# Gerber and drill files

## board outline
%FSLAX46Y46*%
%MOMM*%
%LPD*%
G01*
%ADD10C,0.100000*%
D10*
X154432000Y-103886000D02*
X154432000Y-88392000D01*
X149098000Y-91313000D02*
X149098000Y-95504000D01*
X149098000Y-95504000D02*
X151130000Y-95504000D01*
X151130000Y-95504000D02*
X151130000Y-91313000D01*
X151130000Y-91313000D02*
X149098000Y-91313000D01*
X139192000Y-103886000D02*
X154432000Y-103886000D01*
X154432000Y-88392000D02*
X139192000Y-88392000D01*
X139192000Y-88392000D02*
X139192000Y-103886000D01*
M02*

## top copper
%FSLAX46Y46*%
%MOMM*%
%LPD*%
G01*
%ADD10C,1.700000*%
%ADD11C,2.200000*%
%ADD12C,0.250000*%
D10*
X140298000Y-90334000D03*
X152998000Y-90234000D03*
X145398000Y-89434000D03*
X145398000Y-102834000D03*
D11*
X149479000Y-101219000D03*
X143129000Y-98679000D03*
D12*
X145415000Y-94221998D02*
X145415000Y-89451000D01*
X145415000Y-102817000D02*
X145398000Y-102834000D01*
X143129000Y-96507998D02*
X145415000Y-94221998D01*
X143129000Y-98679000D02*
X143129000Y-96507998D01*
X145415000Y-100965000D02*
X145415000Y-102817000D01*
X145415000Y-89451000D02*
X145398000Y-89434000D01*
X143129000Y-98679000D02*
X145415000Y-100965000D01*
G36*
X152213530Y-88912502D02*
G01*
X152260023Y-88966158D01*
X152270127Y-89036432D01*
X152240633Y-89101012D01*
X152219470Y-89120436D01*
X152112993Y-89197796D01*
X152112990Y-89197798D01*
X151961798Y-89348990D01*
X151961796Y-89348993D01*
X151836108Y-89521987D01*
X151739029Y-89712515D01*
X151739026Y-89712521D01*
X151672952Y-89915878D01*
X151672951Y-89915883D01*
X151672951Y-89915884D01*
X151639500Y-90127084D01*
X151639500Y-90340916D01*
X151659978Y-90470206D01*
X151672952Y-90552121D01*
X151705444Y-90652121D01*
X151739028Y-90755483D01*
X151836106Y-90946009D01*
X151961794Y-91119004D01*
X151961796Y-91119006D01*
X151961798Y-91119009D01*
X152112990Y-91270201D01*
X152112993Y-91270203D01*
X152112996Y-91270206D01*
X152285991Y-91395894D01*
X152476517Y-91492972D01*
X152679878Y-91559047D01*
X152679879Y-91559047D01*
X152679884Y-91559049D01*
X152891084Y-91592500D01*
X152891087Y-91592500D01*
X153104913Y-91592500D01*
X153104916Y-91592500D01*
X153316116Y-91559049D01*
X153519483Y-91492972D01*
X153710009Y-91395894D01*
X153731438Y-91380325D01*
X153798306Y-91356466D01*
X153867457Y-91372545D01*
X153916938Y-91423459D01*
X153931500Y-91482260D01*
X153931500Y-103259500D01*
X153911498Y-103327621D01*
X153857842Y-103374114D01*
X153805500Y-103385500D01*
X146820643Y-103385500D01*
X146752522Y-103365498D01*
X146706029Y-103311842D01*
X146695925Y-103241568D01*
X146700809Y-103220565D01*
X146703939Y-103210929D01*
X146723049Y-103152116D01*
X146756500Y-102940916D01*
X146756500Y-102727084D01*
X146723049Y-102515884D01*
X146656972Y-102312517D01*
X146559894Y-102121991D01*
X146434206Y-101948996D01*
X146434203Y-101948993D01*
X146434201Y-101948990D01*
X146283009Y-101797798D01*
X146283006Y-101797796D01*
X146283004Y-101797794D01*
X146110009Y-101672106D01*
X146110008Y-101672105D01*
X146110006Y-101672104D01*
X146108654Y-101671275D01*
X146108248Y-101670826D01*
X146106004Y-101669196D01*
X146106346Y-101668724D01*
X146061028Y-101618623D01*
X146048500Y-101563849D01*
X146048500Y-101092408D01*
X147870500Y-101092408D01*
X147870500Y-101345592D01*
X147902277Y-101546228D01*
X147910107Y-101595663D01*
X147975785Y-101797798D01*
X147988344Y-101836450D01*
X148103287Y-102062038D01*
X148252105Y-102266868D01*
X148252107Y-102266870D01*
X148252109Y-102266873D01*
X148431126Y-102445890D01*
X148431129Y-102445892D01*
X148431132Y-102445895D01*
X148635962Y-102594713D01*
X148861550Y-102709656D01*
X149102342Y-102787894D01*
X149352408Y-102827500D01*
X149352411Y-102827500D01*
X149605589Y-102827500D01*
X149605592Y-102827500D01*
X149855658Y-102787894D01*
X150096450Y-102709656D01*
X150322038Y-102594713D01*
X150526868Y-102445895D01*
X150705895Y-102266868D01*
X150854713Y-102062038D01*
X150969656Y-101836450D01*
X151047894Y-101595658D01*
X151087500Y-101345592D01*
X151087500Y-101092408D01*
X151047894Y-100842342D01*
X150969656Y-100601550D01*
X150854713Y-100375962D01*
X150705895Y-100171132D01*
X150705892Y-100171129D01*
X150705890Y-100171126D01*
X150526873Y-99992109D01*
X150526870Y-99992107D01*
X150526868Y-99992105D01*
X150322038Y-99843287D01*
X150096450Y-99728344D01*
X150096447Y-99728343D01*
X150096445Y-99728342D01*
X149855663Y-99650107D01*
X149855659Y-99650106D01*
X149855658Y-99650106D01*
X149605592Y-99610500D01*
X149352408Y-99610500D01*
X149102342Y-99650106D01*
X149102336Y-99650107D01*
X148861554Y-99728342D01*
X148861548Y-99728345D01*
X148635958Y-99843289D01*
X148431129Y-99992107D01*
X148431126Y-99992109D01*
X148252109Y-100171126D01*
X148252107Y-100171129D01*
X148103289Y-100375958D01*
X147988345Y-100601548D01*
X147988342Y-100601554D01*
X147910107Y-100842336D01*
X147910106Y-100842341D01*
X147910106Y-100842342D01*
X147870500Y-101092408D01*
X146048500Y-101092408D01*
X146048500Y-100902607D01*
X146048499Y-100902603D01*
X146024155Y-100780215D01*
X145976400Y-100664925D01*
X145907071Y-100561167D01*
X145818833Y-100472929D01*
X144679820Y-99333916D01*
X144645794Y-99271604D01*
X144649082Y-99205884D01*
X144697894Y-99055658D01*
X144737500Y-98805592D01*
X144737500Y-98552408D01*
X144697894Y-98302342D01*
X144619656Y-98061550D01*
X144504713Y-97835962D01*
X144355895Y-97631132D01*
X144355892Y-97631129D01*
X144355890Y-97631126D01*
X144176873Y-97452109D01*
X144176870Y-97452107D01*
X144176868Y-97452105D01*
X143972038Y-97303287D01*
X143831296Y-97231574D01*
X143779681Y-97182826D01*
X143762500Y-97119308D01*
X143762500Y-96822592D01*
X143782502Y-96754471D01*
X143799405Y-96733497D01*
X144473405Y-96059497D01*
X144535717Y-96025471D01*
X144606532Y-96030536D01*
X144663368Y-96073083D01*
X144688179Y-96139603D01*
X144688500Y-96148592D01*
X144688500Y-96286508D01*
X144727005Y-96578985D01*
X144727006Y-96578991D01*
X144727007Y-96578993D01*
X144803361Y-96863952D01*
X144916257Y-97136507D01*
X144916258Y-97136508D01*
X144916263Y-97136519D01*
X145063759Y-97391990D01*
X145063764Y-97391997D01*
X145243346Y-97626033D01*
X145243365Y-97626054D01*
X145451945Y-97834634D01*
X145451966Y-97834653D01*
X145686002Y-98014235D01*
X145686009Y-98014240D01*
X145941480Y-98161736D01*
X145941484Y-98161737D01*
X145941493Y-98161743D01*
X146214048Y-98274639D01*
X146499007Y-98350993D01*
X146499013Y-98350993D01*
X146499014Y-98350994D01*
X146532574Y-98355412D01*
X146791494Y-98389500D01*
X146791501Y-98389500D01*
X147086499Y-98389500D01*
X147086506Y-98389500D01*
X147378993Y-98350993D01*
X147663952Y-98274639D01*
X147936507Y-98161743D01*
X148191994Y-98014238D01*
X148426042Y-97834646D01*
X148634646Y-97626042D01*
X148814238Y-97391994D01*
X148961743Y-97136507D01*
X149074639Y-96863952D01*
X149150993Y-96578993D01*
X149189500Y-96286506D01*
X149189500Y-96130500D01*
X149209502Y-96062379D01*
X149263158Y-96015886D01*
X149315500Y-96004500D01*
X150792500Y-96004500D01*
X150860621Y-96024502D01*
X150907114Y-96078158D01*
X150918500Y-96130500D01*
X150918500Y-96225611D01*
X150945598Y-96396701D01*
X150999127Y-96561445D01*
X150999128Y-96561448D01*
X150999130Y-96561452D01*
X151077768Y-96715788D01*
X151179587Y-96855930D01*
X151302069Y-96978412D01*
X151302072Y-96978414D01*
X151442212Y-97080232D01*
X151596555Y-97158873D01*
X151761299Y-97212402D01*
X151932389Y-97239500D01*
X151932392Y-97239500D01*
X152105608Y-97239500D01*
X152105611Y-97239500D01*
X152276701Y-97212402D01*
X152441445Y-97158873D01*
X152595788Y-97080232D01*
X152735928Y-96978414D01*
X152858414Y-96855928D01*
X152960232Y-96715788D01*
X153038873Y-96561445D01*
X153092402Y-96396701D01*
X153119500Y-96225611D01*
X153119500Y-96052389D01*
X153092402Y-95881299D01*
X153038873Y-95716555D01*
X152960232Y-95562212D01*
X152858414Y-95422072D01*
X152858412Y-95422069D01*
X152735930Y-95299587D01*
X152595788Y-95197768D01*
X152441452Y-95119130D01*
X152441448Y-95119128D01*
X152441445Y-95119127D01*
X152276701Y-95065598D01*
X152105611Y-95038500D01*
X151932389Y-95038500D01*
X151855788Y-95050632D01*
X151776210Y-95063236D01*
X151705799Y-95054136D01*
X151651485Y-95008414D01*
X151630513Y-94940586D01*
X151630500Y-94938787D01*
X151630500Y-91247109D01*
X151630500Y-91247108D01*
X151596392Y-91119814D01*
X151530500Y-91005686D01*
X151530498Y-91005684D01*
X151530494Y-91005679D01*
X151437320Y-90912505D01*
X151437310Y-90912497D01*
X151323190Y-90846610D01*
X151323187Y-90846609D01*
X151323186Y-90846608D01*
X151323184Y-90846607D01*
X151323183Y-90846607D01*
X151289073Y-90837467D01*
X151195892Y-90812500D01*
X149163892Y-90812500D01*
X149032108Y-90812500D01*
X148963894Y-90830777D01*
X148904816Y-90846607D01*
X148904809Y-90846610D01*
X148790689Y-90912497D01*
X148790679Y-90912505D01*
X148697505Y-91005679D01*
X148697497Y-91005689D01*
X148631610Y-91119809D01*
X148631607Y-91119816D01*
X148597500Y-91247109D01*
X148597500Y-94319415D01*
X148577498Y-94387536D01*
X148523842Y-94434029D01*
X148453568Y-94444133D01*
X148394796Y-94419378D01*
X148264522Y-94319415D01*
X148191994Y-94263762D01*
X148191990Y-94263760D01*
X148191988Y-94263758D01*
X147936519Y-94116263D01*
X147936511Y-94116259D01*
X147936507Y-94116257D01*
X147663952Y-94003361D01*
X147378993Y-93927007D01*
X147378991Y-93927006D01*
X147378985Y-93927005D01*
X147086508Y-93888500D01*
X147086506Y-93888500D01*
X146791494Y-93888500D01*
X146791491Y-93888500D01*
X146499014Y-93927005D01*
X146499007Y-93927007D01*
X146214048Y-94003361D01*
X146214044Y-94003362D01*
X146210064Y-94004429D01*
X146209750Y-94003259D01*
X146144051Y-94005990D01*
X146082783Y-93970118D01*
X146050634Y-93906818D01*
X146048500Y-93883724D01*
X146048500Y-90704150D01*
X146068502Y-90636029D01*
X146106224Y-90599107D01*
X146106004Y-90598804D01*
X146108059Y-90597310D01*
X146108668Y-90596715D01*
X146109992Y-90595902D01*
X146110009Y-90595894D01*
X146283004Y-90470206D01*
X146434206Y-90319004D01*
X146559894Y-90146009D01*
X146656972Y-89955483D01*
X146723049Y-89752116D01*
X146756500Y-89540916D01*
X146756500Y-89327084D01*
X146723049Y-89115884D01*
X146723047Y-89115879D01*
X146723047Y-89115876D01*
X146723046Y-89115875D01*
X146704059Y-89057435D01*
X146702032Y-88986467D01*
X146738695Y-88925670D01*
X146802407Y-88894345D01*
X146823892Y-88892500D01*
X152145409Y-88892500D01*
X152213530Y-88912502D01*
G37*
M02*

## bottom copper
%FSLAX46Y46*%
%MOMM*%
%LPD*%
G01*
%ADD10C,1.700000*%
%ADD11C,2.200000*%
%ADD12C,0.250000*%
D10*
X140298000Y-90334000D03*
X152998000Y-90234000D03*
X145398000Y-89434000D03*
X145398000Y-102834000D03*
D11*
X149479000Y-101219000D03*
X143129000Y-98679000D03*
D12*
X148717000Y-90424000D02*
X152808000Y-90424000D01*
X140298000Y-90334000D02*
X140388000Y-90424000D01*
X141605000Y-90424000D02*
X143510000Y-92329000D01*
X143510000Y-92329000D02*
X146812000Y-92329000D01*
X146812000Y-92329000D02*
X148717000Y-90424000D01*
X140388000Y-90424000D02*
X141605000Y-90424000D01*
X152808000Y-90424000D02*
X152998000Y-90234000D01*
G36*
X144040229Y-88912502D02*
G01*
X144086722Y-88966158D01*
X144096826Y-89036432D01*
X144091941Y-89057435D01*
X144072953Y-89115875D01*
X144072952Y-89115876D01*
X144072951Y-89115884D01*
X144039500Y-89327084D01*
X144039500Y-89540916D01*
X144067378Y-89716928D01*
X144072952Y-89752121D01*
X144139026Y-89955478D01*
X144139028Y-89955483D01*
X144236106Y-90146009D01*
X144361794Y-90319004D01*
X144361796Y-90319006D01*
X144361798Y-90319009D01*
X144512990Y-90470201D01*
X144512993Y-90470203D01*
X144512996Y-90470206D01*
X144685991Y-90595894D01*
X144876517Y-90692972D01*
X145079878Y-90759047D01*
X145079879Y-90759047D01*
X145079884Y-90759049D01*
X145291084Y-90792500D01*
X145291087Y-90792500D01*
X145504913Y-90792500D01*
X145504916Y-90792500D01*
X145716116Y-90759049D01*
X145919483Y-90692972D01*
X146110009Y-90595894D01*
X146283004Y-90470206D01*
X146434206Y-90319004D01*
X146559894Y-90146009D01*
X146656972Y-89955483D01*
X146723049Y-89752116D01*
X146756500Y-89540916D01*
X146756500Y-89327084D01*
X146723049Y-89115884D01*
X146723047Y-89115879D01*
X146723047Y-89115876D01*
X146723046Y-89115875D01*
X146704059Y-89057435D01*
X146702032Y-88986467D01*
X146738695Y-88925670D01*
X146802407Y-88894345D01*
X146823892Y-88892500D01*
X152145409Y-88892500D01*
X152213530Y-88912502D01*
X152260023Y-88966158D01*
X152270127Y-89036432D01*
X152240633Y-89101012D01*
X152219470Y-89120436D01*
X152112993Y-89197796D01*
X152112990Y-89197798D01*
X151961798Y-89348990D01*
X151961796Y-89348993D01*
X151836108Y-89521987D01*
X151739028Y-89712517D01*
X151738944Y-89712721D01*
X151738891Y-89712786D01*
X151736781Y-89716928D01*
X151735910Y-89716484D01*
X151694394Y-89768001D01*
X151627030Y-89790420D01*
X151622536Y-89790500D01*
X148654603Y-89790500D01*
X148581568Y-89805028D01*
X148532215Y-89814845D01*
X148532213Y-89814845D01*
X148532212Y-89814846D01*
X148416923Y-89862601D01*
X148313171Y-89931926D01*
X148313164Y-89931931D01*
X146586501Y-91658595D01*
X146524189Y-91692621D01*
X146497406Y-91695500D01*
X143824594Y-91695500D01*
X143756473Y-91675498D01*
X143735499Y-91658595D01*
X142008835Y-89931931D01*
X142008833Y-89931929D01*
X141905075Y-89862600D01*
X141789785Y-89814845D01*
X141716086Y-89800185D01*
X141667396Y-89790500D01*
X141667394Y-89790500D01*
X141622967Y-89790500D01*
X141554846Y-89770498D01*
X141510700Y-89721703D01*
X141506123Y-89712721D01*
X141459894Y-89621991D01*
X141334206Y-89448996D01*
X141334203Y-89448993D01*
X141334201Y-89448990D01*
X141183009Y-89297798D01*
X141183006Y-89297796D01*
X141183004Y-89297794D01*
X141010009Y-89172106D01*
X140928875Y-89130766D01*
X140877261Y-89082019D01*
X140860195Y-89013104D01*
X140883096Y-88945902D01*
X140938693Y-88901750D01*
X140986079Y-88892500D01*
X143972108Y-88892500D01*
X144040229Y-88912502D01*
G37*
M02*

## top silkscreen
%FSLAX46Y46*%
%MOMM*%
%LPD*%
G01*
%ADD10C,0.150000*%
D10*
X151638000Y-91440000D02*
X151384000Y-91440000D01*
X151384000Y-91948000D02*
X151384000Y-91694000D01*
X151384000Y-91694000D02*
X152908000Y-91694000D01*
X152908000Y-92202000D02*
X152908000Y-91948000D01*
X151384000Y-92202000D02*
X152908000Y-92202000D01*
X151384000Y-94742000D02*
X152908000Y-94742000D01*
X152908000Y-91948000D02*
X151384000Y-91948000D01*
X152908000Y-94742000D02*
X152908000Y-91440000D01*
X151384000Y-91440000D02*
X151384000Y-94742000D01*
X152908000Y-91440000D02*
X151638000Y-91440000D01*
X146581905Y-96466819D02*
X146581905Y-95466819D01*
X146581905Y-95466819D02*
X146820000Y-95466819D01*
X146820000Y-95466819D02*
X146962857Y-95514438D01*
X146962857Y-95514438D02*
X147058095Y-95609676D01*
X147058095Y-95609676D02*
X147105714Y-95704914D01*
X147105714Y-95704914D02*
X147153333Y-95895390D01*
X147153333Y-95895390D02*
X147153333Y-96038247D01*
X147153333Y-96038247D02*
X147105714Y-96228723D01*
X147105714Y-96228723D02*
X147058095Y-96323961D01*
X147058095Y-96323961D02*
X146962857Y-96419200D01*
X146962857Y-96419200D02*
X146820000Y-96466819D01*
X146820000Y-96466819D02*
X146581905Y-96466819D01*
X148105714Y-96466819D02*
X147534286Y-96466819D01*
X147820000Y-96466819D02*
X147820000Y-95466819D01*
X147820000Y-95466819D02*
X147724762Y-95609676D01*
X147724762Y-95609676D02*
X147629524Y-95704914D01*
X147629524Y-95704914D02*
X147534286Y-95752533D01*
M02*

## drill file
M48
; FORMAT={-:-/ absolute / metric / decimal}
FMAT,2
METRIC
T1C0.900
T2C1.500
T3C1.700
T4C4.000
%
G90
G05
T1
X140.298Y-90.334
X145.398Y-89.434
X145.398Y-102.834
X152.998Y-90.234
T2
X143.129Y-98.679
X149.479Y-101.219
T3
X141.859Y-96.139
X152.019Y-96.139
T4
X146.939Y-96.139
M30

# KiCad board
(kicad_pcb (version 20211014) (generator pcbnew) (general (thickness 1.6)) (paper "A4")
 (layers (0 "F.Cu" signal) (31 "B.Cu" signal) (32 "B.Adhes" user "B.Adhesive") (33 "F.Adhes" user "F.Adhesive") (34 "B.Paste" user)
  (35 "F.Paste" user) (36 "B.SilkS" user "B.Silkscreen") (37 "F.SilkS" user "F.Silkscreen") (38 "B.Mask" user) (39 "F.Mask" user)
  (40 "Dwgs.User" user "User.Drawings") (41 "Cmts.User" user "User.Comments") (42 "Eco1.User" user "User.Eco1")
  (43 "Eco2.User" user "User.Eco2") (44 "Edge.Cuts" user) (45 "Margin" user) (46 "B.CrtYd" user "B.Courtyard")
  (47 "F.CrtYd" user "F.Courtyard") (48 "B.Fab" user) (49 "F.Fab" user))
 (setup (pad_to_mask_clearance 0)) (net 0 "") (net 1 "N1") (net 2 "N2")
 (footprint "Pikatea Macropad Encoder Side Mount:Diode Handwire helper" (layer "F.Cu") (at 149.098 94.234)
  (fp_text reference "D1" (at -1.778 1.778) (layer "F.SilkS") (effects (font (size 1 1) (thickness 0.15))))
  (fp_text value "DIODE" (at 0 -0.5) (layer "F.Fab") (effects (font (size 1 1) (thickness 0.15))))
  (pad "1" thru_hole circle locked (at -8.8 -3.9 90) (size 1.7 1.7) (drill 0.9) (layers *.Cu *.Mask) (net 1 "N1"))
  (pad "1" thru_hole circle locked (at 3.9 -4 90) (size 1.7 1.7) (drill 0.9) (layers *.Cu *.Mask) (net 1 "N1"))
  (pad "2" thru_hole circle locked (at -3.7 -4.8 90) (size 1.7 1.7) (drill 0.9) (layers *.Cu *.Mask) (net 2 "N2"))
  (pad "2" thru_hole circle locked (at -3.7 8.6 90) (size 1.7 1.7) (drill 0.9) (layers *.Cu *.Mask) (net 2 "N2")))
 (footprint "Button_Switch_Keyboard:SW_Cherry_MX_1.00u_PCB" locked (layer "B.Cu") (at 149.479 101.219)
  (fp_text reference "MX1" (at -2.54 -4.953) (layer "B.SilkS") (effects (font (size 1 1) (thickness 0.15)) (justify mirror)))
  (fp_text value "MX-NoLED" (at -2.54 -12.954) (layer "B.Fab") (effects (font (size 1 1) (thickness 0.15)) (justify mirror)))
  (pad "" np_thru_hole circle locked (at 2.54 -5.08) (size 1.7 1.7) (drill 1.7) (layers *.Cu *.Mask))
  (pad "" np_thru_hole circle locked (at -2.54 -5.08) (size 4 4) (drill 4) (layers *.Cu *.Mask))
  (pad "" np_thru_hole circle locked (at -7.62 -5.08) (size 1.7 1.7) (drill 1.7) (layers *.Cu *.Mask))
  (pad "1" thru_hole circle locked (at 0 0) (size 2.2 2.2) (drill 1.5) (layers *.Cu *.Mask))
  (pad "2" thru_hole circle locked (at -6.35 -2.54) (size 2.2 2.2) (drill 1.5) (layers *.Cu *.Mask) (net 2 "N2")))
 (gr_line (start 151.638 91.44) (end 151.384 91.44) (layer "F.SilkS") (width 0.15))
 (gr_line (start 151.384 91.948) (end 151.384 91.694) (layer "F.SilkS") (width 0.15))
 (gr_line (start 151.384 91.694) (end 152.908 91.694) (layer "F.SilkS") (width 0.15))
 (gr_line (start 152.908 92.202) (end 152.908 91.948) (layer "F.SilkS") (width 0.15))
 (gr_line (start 151.384 92.202) (end 152.908 92.202) (layer "F.SilkS") (width 0.15))
 (gr_line (start 151.384 94.742) (end 152.908 94.742) (layer "F.SilkS") (width 0.15))
 (gr_line (start 152.908 91.948) (end 151.384 91.948) (layer "F.SilkS") (width 0.15))
 (gr_line (start 152.908 94.742) (end 152.908 91.44) (layer "F.SilkS") (width 0.15))
 (gr_line (start 151.384 91.44) (end 151.384 94.742) (layer "F.SilkS") (width 0.15))
 (gr_line (start 152.908 91.44) (end 151.638 91.44) (layer "F.SilkS") (width 0.15))
 (gr_line (start 154.432 103.886) (end 154.432 88.392) (layer "Edge.Cuts") (width 0.1))
 (gr_line (start 149.098 91.313) (end 149.098 95.504) (layer "Edge.Cuts") (width 0.1))
 (gr_line (start 149.098 95.504) (end 151.13 95.504) (layer "Edge.Cuts") (width 0.1))
 (gr_line (start 151.13 95.504) (end 151.13 91.313) (layer "Edge.Cuts") (width 0.1))
 (gr_line (start 151.13 91.313) (end 149.098 91.313) (layer "Edge.Cuts") (width 0.1))
 (gr_line (start 139.192 103.886) (end 154.432 103.886) (layer "Edge.Cuts") (width 0.1))
 (gr_line (start 154.432 88.392) (end 139.192 88.392) (layer "Edge.Cuts") (width 0.1))
 (gr_line (start 139.192 88.392) (end 139.192 103.886) (layer "Edge.Cuts") (width 0.1))
 (segment (start 145.415 94.221998) (end 145.415 89.451) (width 0.25) (layer "F.Cu") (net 2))
 (segment (start 145.415 102.817) (end 145.398 102.834) (width 0.25) (layer "F.Cu") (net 2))
 (segment (start 143.129 96.507998) (end 145.415 94.221998) (width 0.25) (layer "F.Cu") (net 2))
 (segment (start 143.129 98.679) (end 143.129 96.507998) (width 0.25) (layer "F.Cu") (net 2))
 (segment (start 145.415 100.965) (end 145.415 102.817) (width 0.25) (layer "F.Cu") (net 2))
 (segment (start 145.415 89.451) (end 145.398 89.434) (width 0.25) (layer "F.Cu") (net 2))
 (segment (start 143.129 98.679) (end 145.415 100.965) (width 0.25) (layer "F.Cu") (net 2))
 (segment (start 148.717 90.424) (end 152.808 90.424) (width 0.25) (layer "B.Cu") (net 1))
 (segment (start 140.298 90.334) (end 140.388 90.424) (width 0.25) (layer "B.Cu") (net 1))
 (segment (start 141.605 90.424) (end 143.51 92.329) (width 0.25) (layer "B.Cu") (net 1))
 (segment (start 143.51 92.329) (end 146.812 92.329) (width 0.25) (layer "B.Cu") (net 1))
 (segment (start 146.812 92.329) (end 148.717 90.424) (width 0.25) (layer "B.Cu") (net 1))
 (segment (start 140.388 90.424) (end 141.605 90.424) (width 0.25) (layer "B.Cu") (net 1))
 (segment (start 152.808 90.424) (end 152.998 90.234) (width 0.25) (layer "B.Cu") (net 1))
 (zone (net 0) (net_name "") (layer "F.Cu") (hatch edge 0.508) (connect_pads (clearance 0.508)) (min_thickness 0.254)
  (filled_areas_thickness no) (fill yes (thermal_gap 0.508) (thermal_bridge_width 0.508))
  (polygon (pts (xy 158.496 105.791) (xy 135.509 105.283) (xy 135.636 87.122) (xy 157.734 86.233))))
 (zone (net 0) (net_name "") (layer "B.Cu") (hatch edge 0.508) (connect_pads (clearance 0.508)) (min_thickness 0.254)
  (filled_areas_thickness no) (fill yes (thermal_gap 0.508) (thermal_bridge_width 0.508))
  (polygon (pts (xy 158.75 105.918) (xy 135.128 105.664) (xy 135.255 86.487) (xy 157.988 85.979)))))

